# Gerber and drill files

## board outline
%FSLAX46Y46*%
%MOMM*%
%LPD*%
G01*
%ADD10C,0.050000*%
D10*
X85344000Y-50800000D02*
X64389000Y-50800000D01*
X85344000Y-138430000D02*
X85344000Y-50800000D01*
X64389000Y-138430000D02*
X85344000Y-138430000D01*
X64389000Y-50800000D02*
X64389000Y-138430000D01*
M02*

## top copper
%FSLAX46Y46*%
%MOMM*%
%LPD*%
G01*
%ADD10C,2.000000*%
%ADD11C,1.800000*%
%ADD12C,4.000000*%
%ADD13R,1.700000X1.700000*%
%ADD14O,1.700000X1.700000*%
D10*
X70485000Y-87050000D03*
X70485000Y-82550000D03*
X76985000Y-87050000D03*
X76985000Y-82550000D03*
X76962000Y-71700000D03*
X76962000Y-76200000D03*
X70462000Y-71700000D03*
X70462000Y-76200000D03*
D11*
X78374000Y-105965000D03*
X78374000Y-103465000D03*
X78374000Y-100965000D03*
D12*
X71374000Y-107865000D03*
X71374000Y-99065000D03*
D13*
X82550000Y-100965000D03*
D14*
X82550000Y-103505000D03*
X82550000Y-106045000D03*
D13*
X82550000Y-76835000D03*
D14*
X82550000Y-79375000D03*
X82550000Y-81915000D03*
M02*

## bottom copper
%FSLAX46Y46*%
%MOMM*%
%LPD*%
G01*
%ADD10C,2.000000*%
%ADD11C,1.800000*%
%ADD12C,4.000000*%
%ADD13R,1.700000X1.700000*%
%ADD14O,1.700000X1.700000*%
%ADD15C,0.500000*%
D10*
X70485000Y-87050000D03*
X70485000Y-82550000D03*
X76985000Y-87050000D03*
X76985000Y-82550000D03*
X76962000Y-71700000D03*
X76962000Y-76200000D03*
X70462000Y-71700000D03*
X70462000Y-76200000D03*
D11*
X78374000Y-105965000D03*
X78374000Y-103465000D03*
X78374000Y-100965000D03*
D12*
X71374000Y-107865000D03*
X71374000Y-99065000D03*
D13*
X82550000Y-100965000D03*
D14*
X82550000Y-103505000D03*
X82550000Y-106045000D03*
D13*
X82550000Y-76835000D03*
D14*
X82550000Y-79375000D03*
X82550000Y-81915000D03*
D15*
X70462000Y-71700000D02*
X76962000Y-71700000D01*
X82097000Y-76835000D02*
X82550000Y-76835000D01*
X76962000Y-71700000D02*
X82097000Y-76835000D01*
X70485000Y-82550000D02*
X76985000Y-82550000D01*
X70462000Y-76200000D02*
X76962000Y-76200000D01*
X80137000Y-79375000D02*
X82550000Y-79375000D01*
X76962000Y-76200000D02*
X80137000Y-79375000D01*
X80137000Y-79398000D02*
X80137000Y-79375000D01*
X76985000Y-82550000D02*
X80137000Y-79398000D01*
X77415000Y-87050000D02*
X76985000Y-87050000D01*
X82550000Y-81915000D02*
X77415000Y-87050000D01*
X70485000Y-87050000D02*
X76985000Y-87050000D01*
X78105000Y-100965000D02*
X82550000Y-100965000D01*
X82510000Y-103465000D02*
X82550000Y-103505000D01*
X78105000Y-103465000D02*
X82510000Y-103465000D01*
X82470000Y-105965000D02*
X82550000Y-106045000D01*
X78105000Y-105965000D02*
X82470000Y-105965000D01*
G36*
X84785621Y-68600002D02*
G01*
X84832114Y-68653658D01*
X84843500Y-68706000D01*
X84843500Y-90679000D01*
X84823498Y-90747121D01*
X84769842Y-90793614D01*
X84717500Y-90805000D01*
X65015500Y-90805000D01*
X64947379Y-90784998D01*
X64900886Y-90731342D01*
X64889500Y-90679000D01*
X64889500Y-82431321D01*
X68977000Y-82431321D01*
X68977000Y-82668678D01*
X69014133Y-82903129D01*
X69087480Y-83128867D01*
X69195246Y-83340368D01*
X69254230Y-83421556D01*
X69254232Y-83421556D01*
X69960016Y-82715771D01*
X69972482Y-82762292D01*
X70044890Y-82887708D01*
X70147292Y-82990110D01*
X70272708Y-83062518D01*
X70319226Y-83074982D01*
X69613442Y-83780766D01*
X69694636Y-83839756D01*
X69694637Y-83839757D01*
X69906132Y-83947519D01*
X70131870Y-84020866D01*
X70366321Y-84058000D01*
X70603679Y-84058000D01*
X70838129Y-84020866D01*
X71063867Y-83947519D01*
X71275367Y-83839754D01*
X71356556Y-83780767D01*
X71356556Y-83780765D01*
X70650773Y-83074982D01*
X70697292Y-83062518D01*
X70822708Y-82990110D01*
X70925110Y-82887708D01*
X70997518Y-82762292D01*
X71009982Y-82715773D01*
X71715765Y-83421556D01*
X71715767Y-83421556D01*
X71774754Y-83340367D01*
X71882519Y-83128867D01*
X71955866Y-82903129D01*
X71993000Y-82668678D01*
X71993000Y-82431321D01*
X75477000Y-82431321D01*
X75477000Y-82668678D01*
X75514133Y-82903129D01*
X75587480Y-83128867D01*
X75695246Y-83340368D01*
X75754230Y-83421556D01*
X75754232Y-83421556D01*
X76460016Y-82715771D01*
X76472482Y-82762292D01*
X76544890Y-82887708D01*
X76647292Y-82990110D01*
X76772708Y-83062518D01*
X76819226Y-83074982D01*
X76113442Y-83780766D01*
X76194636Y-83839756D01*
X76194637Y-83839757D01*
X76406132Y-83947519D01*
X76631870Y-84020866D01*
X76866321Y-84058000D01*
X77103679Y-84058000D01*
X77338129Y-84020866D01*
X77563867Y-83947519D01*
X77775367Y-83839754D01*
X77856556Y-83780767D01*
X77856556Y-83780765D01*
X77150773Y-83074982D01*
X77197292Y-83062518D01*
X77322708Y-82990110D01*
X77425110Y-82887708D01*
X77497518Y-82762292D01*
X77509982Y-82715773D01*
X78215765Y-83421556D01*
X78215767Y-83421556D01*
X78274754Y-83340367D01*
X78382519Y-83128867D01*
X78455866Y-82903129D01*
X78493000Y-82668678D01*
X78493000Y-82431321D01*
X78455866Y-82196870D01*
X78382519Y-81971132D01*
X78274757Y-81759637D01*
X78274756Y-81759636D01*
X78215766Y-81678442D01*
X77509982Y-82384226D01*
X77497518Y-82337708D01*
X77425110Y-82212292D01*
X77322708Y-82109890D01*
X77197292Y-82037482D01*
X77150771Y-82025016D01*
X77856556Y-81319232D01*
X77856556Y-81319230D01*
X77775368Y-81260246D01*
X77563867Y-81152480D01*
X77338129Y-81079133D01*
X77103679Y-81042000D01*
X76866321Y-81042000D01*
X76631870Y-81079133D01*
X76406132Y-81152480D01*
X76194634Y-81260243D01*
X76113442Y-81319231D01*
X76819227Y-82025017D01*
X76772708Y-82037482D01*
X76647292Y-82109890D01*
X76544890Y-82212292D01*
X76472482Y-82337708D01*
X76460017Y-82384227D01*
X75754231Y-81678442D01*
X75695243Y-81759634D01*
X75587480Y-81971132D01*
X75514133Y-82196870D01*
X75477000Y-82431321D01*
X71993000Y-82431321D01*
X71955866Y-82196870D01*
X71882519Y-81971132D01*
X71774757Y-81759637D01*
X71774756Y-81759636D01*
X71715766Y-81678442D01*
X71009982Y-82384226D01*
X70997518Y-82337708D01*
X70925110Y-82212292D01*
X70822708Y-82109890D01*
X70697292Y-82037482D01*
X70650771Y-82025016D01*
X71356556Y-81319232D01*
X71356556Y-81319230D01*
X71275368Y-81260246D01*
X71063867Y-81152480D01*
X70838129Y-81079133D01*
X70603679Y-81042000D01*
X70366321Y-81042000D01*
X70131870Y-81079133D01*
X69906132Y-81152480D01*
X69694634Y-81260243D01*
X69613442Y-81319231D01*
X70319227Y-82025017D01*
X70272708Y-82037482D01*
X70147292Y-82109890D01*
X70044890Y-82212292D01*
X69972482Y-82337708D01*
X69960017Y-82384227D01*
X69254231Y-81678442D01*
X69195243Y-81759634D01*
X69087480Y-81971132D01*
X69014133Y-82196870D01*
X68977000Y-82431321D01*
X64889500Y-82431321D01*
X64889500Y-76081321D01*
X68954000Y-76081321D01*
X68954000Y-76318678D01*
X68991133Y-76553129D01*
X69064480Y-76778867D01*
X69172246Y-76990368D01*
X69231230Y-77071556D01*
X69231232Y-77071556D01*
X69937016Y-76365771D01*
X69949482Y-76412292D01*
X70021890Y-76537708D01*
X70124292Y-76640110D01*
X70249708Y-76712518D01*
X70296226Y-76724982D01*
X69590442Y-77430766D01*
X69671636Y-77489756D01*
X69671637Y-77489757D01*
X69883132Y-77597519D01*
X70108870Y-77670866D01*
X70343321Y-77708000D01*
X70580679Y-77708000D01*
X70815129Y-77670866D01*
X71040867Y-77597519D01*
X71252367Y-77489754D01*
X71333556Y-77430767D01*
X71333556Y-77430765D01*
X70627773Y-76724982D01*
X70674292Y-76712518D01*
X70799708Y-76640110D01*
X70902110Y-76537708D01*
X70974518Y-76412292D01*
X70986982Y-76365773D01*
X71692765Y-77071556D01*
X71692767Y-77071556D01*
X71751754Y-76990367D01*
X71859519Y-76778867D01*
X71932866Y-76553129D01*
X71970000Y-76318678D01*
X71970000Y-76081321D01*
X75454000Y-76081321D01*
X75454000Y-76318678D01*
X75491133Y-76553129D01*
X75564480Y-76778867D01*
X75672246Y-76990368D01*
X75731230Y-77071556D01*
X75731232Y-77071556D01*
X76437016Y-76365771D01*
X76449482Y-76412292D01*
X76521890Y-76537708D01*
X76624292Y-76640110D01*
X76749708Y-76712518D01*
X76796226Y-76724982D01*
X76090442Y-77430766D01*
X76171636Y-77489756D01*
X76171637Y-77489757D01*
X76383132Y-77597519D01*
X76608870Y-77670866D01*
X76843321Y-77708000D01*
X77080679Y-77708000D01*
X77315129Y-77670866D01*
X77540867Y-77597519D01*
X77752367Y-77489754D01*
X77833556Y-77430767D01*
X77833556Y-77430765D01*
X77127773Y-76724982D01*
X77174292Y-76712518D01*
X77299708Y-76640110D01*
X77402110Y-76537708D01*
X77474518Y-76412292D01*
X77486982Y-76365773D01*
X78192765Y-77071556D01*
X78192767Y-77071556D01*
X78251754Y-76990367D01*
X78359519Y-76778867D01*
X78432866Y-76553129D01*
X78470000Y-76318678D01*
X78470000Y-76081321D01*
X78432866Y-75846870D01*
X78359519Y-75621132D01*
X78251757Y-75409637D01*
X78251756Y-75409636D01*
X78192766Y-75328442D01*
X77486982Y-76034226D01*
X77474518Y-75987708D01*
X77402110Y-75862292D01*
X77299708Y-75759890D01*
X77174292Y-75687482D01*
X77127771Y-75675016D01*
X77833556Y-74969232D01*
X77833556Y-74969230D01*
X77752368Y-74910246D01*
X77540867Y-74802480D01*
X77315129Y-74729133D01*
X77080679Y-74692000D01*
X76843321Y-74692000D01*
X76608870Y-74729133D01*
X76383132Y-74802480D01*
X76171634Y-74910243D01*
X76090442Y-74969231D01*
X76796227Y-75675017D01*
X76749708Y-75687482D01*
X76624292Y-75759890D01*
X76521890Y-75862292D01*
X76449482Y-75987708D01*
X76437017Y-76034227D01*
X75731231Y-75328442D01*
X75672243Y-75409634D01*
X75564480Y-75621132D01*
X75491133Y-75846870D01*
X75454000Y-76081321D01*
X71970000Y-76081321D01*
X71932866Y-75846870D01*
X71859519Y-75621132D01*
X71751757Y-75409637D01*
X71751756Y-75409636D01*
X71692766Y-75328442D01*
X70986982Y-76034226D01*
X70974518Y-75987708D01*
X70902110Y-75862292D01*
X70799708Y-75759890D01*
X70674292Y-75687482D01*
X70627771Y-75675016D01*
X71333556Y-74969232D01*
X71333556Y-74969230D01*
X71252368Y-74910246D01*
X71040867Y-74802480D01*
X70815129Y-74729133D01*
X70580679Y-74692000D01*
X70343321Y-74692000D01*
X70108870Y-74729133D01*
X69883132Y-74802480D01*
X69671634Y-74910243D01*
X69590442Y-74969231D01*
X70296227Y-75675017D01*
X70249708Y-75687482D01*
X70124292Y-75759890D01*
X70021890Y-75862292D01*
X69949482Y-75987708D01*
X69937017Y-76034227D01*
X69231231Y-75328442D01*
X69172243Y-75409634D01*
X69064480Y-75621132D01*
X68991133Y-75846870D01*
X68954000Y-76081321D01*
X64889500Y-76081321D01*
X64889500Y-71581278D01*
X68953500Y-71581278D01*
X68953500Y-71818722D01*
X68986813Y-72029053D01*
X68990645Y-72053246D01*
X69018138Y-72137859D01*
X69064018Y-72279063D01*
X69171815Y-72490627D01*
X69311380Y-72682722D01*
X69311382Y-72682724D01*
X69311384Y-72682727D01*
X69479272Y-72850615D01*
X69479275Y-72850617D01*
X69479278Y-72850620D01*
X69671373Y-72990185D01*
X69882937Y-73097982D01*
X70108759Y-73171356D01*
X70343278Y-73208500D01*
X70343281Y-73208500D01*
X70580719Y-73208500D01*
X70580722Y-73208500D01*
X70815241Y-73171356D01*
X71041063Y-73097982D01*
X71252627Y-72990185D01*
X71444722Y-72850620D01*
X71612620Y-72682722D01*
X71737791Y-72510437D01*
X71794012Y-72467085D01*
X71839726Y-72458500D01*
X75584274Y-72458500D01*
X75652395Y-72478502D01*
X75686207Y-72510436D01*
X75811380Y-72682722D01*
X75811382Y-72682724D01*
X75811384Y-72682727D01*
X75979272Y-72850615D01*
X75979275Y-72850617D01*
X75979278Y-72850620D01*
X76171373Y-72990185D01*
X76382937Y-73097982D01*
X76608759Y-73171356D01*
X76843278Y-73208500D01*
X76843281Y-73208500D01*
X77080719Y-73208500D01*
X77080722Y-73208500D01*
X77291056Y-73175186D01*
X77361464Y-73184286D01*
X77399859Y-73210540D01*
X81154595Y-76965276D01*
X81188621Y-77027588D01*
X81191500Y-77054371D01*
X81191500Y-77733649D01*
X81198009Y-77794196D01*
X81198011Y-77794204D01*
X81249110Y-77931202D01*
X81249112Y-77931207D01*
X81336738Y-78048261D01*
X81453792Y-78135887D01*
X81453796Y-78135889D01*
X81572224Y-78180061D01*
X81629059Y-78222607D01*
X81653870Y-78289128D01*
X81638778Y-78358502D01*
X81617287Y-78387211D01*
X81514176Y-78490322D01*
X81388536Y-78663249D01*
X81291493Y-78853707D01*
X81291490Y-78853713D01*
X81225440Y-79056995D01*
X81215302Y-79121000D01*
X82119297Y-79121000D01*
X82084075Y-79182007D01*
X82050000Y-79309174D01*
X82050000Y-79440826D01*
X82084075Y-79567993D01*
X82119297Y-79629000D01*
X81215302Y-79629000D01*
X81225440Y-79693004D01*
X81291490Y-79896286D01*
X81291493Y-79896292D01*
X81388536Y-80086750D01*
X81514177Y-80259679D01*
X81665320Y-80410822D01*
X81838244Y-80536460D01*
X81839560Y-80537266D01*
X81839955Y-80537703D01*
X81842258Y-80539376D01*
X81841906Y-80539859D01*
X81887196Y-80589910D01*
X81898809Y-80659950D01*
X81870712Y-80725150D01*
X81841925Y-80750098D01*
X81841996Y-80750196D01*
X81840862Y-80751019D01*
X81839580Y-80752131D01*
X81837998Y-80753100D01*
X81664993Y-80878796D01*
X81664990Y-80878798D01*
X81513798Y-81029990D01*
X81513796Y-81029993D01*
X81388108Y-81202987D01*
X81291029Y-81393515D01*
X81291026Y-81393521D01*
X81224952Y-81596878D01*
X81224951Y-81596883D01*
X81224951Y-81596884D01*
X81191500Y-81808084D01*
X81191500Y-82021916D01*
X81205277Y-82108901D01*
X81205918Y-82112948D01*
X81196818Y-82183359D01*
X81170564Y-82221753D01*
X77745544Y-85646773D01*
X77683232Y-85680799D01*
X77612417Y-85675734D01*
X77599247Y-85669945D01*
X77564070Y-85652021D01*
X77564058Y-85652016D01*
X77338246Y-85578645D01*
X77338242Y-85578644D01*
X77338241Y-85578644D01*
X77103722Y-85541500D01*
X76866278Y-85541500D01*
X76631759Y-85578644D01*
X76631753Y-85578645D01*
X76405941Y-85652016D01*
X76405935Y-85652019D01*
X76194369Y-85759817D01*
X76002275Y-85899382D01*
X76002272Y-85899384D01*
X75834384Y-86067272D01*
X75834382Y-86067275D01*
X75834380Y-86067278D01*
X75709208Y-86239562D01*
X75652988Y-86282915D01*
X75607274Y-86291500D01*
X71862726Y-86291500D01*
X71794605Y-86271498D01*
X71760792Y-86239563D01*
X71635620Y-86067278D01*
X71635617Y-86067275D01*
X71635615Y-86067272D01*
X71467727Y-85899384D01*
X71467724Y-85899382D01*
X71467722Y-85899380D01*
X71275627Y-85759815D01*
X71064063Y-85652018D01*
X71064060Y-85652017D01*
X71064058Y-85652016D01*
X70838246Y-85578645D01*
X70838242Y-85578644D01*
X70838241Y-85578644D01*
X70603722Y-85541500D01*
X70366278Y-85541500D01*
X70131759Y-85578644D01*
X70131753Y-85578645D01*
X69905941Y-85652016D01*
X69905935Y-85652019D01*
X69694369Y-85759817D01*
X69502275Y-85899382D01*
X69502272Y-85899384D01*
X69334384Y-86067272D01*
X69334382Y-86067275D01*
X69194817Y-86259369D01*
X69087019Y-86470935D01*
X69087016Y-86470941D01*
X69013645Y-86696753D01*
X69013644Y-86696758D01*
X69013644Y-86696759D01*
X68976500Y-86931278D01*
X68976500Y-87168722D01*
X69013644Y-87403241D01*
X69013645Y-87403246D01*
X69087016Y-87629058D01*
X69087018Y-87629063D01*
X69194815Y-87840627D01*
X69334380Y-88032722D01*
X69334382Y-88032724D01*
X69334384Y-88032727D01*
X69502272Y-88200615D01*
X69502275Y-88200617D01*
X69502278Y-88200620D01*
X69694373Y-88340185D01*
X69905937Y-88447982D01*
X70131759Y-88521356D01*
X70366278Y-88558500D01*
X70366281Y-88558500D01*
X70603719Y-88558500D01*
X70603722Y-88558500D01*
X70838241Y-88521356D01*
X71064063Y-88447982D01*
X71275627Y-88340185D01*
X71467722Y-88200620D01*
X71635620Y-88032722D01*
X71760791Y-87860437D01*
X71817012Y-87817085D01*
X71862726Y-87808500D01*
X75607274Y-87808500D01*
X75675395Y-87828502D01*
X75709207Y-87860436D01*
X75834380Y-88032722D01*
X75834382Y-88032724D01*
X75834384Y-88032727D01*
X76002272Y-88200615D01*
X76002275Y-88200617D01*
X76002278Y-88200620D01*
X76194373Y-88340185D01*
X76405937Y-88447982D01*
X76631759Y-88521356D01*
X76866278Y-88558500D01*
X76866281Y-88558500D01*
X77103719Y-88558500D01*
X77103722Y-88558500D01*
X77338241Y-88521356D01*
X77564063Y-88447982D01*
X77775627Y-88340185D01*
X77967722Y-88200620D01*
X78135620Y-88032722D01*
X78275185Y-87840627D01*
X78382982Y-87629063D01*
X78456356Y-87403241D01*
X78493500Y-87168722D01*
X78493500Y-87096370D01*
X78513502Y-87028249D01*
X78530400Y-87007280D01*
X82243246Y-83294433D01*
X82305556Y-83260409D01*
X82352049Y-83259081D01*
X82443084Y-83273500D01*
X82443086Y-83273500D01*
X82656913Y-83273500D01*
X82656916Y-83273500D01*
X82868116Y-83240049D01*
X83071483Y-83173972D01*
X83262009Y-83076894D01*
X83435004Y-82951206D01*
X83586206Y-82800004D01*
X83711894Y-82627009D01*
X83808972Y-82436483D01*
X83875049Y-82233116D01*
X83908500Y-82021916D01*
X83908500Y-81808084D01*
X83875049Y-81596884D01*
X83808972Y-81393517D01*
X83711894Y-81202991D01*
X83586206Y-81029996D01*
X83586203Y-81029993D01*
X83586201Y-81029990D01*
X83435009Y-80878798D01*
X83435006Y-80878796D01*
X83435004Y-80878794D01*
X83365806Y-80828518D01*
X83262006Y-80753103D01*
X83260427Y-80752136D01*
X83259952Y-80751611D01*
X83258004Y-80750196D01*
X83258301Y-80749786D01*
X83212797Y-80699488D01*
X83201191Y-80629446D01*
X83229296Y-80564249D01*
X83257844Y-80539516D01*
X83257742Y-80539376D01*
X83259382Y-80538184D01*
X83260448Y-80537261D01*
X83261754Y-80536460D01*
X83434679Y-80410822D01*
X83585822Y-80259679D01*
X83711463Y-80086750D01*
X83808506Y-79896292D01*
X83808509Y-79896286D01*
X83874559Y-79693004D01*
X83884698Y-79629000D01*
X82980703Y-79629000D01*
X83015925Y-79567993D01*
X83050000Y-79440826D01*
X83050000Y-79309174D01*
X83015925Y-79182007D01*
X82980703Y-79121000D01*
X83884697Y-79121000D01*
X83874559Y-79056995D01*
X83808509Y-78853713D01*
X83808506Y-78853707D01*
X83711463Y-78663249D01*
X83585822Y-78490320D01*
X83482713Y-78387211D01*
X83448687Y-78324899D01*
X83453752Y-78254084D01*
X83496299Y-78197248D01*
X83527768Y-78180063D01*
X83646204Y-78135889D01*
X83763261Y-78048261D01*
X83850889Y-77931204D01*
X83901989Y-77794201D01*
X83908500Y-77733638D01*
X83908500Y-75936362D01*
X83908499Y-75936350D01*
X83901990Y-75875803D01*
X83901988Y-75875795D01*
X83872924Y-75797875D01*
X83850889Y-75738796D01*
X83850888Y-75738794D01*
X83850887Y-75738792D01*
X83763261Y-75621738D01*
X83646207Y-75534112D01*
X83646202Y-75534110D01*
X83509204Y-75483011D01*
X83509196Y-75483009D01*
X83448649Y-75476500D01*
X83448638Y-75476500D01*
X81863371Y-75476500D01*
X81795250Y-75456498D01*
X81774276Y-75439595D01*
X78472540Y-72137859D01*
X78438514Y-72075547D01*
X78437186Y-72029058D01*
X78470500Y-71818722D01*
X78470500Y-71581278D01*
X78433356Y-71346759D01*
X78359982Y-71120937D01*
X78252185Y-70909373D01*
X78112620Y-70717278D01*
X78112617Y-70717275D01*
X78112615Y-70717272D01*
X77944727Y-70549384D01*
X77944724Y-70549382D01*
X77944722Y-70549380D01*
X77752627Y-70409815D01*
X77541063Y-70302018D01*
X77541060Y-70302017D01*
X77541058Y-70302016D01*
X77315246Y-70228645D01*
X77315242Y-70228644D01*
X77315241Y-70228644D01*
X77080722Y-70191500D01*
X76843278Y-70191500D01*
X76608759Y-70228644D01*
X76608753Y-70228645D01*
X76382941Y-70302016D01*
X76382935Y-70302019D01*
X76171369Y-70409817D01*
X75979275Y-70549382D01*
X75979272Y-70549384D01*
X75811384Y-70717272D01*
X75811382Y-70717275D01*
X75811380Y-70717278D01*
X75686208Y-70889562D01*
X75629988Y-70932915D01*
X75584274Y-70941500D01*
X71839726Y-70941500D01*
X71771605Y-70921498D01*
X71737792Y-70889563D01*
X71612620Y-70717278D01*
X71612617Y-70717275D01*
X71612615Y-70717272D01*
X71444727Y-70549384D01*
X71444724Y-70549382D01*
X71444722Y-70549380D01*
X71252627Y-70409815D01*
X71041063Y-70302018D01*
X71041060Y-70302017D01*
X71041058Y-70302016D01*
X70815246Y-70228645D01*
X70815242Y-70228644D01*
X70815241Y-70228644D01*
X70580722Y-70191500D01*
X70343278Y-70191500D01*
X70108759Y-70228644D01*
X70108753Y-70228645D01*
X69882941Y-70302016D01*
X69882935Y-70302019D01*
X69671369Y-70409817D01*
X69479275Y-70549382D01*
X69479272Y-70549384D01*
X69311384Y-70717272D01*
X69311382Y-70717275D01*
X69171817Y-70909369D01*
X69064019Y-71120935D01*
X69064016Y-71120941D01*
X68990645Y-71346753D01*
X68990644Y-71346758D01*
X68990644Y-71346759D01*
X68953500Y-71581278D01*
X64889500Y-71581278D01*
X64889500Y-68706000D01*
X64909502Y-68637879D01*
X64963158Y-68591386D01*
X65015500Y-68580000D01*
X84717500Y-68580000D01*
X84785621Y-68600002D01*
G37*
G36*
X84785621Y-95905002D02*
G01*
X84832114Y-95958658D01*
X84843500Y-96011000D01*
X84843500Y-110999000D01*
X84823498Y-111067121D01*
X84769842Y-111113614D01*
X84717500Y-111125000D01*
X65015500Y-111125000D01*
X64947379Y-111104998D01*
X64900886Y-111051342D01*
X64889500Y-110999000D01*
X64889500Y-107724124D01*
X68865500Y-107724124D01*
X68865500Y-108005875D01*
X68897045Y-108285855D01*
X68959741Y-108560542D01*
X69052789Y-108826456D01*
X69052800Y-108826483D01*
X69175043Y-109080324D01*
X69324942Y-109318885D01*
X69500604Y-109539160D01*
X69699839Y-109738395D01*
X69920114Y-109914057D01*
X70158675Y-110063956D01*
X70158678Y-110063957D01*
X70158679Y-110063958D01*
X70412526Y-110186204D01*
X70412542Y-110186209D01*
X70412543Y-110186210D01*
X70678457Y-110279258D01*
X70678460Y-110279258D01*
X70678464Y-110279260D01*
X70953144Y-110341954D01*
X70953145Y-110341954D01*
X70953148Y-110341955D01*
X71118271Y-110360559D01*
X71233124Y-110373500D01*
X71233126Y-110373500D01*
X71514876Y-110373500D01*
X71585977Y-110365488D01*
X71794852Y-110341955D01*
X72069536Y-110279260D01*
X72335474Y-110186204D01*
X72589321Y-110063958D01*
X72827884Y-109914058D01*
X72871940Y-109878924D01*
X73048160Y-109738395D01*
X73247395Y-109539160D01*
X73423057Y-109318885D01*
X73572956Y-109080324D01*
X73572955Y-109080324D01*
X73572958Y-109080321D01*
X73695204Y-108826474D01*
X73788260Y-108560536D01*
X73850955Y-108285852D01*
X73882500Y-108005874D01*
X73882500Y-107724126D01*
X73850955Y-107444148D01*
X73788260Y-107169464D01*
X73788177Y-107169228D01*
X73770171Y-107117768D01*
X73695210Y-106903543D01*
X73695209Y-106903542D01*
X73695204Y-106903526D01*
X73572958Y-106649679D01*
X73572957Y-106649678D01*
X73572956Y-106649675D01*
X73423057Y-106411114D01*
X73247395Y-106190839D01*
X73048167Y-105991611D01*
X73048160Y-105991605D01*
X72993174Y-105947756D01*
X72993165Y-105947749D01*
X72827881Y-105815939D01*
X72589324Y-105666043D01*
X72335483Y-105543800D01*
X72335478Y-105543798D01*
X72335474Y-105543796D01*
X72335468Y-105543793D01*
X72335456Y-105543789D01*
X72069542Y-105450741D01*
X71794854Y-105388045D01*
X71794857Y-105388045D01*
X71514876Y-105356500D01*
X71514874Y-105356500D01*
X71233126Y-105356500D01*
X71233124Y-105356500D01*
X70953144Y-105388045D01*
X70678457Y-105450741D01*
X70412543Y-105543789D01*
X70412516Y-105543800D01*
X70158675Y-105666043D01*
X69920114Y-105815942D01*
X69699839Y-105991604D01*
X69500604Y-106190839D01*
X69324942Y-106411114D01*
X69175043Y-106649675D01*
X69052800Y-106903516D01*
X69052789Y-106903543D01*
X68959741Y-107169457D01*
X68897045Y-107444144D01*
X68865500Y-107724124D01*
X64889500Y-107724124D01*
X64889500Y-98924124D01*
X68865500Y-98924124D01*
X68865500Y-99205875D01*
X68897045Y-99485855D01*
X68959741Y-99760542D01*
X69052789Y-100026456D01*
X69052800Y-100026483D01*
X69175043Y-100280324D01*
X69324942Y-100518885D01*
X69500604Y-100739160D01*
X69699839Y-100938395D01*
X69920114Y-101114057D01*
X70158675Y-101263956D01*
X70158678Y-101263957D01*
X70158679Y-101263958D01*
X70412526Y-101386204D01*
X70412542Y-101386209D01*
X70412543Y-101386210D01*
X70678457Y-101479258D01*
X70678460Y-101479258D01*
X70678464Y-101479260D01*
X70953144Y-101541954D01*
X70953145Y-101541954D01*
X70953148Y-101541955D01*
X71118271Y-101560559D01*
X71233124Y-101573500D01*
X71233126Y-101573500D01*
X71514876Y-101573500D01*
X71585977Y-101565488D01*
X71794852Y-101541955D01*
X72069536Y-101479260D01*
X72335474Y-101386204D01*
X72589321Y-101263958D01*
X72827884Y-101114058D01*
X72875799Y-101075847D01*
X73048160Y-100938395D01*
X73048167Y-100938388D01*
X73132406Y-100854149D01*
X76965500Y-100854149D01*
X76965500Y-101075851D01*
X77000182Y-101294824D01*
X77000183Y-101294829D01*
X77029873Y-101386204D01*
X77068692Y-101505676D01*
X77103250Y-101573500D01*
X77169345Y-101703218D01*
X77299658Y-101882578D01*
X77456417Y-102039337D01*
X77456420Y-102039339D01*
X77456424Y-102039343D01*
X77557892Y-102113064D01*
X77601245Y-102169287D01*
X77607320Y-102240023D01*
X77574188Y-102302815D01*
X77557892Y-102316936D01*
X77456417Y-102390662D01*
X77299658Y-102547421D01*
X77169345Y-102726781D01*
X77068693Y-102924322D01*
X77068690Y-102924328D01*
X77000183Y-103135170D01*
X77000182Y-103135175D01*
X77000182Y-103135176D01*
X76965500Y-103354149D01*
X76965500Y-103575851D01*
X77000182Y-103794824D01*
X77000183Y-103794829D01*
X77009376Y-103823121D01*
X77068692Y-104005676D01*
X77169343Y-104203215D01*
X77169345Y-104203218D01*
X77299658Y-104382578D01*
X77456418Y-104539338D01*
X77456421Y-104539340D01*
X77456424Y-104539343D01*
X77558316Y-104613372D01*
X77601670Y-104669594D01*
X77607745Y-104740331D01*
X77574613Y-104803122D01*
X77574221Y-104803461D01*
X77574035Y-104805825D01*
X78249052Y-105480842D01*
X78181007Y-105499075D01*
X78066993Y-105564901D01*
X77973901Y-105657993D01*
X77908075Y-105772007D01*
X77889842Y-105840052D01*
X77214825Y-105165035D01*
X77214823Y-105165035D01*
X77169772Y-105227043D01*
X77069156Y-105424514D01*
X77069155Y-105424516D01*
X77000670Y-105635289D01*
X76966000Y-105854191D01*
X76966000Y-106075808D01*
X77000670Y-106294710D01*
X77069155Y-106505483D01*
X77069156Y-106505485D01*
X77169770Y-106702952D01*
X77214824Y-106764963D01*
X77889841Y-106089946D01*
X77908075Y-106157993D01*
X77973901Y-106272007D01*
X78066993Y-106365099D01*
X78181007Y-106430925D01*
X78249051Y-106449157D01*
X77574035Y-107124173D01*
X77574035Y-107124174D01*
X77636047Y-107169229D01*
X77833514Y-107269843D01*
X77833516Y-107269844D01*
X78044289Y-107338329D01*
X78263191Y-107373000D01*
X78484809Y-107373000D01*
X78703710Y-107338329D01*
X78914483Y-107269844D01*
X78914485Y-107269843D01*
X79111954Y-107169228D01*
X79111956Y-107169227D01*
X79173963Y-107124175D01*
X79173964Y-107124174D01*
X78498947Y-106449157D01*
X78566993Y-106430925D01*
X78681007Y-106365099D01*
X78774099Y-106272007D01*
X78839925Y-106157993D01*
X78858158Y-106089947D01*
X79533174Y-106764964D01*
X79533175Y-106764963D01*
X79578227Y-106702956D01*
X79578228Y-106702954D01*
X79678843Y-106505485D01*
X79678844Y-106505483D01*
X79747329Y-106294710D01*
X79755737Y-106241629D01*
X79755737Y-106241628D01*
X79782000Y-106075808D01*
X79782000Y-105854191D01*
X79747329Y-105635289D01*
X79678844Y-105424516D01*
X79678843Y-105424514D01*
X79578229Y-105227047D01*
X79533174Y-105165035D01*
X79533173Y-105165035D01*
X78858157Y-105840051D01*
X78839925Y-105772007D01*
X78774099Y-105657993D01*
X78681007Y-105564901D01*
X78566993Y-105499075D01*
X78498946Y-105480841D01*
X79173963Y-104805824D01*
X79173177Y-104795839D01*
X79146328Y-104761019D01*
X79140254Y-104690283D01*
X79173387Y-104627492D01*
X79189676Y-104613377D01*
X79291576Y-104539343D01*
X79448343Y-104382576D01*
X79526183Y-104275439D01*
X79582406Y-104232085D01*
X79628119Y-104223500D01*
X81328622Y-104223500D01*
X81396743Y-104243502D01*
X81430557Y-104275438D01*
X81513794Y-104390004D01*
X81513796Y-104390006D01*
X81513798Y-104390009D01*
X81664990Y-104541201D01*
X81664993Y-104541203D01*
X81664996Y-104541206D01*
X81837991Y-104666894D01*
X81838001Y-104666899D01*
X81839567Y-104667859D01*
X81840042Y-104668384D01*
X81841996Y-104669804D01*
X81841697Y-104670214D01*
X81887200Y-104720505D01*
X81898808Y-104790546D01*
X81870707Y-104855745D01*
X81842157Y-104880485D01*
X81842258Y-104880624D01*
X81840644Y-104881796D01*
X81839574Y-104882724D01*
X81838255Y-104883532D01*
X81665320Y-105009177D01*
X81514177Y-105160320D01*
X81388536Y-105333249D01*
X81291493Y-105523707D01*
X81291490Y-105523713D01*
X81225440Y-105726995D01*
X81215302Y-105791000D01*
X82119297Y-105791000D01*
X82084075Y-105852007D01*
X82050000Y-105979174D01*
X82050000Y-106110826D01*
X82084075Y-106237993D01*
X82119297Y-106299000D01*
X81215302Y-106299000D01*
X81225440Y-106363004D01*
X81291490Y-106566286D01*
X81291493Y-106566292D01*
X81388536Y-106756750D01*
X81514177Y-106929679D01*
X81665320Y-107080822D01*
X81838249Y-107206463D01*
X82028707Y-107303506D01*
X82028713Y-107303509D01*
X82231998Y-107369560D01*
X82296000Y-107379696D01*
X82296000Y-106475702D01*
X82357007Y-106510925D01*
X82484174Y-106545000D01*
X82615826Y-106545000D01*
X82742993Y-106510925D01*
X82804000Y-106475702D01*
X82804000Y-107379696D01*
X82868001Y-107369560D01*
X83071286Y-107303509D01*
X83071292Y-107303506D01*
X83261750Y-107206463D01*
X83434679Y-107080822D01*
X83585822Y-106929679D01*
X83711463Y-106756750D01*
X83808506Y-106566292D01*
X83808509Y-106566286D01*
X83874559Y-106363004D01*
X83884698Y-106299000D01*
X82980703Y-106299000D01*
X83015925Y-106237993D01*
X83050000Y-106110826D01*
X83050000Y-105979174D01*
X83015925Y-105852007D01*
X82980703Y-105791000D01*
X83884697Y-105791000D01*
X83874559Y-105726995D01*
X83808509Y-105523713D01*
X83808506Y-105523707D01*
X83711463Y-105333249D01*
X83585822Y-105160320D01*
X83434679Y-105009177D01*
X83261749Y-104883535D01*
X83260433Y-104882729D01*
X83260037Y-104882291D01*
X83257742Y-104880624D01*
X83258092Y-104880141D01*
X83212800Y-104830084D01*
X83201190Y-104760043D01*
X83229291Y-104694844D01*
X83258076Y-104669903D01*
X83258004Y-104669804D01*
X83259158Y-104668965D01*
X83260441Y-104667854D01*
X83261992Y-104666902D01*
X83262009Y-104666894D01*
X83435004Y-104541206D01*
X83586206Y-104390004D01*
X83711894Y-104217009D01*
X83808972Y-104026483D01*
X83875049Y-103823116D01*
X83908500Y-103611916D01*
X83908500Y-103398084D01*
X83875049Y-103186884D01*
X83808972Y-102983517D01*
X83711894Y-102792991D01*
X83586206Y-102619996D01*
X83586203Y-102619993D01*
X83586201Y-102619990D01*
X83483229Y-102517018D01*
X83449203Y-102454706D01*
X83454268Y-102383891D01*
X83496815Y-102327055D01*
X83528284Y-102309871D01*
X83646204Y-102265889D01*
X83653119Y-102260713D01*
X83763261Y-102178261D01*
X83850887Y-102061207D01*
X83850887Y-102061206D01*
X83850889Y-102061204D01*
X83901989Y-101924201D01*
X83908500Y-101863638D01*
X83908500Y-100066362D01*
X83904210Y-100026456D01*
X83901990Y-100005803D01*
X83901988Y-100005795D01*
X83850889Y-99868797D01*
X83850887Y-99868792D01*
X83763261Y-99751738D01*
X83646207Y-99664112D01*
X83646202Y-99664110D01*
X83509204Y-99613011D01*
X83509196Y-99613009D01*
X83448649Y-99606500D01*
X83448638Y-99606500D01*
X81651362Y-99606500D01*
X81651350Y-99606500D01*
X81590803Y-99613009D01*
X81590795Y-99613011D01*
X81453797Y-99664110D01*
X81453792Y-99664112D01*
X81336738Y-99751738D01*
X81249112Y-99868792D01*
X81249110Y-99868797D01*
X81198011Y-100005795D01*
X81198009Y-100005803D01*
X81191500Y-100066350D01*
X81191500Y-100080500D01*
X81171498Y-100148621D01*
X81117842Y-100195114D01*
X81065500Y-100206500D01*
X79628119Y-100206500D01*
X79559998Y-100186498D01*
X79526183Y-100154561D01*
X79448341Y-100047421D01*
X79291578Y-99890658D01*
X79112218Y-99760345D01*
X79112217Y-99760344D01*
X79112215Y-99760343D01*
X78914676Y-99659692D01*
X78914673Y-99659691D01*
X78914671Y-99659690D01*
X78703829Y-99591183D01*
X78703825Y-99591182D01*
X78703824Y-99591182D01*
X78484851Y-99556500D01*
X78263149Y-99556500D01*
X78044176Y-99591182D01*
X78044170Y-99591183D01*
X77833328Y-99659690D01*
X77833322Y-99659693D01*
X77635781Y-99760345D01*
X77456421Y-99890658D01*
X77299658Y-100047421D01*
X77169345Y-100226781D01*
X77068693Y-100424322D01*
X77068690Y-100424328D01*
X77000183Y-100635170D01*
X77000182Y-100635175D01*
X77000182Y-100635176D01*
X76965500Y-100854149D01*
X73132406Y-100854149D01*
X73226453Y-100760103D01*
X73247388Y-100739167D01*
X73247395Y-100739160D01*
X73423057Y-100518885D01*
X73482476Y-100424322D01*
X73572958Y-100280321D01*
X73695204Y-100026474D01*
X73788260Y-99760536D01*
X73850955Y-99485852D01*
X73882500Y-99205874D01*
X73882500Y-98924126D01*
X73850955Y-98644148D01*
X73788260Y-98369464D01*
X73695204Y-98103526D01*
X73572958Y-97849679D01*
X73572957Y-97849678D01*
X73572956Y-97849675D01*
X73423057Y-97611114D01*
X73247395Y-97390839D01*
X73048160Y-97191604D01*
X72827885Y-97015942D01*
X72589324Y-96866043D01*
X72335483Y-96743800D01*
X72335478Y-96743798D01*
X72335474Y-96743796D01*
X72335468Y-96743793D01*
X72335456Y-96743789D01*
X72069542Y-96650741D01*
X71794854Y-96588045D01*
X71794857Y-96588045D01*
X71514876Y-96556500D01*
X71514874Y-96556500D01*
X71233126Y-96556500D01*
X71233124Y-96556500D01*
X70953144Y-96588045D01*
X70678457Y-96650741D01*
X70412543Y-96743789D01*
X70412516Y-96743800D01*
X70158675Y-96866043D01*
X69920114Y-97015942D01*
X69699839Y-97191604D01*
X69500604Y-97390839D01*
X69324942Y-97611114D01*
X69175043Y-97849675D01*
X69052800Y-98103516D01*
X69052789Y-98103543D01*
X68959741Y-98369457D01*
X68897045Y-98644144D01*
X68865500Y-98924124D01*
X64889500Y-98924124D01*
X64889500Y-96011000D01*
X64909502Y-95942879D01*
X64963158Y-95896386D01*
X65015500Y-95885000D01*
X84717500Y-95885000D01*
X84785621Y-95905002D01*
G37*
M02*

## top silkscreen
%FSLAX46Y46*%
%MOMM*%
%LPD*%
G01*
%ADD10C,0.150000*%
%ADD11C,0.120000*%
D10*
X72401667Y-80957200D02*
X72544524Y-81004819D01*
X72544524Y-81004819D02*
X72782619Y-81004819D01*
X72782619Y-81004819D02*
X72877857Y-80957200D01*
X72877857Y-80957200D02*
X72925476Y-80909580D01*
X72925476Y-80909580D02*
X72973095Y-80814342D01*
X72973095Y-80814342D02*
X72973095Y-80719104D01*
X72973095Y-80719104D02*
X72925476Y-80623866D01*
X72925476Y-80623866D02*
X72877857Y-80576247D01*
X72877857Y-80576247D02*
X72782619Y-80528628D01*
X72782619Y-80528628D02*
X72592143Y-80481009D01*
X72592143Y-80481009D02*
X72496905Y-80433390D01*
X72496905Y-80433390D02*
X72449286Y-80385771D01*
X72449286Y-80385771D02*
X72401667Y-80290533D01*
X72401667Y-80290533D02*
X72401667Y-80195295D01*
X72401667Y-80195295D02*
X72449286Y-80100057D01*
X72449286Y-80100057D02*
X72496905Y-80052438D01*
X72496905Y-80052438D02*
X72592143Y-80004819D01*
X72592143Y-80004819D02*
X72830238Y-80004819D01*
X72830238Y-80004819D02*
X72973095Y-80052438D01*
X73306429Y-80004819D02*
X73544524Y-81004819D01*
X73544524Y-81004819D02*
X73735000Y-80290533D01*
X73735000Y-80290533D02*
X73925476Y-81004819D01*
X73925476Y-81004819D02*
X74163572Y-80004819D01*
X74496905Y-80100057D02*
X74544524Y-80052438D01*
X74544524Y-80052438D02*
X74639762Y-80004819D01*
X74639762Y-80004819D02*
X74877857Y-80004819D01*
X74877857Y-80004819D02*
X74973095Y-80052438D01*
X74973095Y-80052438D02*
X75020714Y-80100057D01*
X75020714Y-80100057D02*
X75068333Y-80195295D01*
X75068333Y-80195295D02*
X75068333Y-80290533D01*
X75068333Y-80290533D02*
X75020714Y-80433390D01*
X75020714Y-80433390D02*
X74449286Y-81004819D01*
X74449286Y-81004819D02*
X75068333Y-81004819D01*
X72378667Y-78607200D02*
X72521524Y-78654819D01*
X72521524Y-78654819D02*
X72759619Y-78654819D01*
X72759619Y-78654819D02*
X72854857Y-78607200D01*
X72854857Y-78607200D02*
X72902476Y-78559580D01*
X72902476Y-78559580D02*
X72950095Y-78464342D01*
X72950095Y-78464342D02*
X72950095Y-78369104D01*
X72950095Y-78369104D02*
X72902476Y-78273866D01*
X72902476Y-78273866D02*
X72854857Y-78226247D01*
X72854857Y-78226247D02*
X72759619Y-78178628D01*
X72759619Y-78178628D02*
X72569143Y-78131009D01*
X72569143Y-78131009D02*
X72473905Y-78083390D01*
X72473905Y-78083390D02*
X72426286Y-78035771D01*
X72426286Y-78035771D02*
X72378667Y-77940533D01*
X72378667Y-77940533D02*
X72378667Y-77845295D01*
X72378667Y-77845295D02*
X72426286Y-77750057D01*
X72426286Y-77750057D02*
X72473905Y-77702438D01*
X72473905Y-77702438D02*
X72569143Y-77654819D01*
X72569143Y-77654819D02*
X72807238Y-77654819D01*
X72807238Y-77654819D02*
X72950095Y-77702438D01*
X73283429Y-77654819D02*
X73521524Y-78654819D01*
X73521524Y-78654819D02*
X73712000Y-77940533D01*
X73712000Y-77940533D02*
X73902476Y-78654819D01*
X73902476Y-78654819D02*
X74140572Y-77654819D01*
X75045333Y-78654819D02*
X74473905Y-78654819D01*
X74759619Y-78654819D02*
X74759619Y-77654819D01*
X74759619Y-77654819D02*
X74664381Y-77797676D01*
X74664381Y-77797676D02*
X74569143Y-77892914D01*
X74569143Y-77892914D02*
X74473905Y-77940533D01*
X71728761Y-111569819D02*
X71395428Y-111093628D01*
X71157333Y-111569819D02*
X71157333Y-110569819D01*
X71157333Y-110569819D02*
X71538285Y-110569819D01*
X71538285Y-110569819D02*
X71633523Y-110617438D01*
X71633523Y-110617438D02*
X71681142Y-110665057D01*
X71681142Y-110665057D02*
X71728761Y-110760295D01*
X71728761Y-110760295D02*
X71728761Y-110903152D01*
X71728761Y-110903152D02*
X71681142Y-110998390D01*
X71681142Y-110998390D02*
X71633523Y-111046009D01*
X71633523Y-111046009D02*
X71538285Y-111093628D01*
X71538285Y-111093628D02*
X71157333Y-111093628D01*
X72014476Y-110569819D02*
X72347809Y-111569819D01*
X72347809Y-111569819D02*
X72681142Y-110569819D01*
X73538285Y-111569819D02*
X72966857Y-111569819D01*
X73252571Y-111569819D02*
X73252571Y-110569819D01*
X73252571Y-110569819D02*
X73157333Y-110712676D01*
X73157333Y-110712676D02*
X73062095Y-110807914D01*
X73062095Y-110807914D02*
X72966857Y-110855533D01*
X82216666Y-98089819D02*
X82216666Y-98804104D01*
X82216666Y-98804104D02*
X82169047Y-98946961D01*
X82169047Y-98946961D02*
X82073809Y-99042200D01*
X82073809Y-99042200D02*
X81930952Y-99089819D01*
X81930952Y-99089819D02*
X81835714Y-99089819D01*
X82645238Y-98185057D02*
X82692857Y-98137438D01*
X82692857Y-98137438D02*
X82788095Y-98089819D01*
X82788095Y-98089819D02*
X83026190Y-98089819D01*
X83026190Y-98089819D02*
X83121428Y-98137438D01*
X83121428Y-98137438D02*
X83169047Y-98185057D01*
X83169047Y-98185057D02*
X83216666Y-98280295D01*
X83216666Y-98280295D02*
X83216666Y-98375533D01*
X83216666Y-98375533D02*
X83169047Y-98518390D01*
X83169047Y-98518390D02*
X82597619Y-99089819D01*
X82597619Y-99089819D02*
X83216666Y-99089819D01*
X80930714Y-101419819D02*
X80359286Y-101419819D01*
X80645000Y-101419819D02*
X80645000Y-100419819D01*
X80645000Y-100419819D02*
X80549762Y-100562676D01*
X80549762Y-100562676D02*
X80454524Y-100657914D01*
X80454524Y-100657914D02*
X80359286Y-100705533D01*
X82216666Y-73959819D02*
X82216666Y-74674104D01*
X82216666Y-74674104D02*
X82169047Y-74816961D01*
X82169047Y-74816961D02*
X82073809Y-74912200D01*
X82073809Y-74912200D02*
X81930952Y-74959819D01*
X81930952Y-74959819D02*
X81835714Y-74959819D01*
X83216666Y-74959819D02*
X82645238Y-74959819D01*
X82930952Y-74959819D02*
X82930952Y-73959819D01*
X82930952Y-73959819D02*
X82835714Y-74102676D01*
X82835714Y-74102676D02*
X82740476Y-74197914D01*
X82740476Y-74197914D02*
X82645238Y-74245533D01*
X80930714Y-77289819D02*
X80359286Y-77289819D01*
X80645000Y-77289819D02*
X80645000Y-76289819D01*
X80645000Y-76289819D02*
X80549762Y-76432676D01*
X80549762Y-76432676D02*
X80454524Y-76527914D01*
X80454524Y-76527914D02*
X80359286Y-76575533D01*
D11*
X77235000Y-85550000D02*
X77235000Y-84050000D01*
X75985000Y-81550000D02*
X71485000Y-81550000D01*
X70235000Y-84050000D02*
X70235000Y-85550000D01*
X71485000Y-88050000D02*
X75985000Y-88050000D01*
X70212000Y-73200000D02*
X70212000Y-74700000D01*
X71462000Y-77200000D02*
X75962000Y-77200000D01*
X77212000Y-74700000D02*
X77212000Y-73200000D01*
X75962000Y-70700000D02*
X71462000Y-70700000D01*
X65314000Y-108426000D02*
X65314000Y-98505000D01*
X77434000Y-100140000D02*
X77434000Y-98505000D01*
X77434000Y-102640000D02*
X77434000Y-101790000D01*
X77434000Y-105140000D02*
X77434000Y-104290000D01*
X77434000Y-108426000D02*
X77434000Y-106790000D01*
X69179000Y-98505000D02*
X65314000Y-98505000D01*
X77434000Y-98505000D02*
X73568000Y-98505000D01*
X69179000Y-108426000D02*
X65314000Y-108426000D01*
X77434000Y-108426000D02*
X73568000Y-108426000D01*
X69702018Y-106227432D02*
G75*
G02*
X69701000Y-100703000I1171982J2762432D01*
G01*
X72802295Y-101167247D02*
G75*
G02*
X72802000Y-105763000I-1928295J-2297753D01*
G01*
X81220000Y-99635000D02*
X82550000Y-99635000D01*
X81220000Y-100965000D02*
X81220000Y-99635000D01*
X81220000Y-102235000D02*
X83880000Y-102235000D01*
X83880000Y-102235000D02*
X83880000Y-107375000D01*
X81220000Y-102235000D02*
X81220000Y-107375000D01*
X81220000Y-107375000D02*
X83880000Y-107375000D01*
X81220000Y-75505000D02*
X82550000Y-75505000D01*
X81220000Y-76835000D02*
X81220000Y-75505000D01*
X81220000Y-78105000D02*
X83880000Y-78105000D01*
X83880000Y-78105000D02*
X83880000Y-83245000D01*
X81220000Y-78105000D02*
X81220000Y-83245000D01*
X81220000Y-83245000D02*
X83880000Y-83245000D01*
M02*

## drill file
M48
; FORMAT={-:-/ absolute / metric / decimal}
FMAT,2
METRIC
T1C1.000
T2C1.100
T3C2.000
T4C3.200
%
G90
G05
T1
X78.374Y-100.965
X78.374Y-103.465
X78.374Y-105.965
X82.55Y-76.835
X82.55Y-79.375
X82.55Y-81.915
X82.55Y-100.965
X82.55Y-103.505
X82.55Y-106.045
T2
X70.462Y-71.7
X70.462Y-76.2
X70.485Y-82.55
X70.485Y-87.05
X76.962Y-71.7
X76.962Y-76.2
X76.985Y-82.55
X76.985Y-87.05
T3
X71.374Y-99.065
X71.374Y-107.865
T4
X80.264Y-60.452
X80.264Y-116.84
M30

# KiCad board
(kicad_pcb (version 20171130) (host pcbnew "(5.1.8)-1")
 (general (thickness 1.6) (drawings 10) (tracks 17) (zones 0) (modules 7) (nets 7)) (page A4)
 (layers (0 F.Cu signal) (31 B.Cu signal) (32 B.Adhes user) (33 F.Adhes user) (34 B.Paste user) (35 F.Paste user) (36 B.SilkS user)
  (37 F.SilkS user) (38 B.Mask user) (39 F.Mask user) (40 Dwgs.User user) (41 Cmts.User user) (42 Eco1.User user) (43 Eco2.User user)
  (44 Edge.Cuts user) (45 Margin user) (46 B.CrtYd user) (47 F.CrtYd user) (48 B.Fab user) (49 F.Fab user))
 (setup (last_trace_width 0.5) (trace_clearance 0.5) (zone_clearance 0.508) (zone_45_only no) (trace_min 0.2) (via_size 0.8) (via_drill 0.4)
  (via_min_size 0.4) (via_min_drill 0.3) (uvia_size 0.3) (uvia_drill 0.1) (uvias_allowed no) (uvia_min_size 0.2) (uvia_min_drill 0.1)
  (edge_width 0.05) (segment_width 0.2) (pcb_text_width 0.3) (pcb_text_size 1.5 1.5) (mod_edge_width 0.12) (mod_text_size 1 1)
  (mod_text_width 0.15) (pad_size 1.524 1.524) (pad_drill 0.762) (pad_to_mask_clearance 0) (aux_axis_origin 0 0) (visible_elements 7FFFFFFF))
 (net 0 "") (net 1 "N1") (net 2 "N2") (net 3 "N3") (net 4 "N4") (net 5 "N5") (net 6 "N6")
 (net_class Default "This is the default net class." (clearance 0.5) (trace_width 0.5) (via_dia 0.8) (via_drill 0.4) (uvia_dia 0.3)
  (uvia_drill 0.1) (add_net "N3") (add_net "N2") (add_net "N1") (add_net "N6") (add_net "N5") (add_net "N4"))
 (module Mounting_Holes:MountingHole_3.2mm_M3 (layer F.Cu) (at 80.264 116.84)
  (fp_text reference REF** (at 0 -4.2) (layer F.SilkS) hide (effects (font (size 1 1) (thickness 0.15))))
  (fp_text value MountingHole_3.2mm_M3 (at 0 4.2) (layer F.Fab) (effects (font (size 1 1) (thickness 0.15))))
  (pad 1 np_thru_hole circle (at 0 0) (size 3.2 3.2) (drill 3.2) (layers *.Cu *.Mask)))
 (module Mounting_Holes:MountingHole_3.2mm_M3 (layer F.Cu) (at 80.264 60.452)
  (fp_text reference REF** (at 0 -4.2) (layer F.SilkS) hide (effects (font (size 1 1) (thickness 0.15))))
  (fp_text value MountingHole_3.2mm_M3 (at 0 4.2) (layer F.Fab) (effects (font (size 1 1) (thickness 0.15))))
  (pad 1 np_thru_hole circle (at 0 0) (size 3.2 3.2) (drill 3.2) (layers *.Cu *.Mask)))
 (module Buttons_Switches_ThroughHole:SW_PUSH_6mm (layer F.Cu) (at 70.485 82.55)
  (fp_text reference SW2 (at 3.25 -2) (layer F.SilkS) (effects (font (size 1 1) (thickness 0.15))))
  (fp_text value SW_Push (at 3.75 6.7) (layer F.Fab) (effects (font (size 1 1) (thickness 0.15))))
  (fp_line (start 6.75 3) (end 6.75 1.5) (layer F.SilkS) (width 0.12))
  (fp_line (start 5.5 -1) (end 1 -1) (layer F.SilkS) (width 0.12))
  (fp_line (start -0.25 1.5) (end -0.25 3) (layer F.SilkS) (width 0.12))
  (fp_line (start 1 5.5) (end 5.5 5.5) (layer F.SilkS) (width 0.12))
  (pad 2 thru_hole circle (at 0 4.5 90) (size 2 2) (drill 1.1) (layers *.Cu *.Mask) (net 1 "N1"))
  (pad 1 thru_hole circle (at 0 0 90) (size 2 2) (drill 1.1) (layers *.Cu *.Mask) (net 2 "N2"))
  (pad 2 thru_hole circle (at 6.5 4.5 90) (size 2 2) (drill 1.1) (layers *.Cu *.Mask) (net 1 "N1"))
  (pad 1 thru_hole circle (at 6.5 0 90) (size 2 2) (drill 1.1) (layers *.Cu *.Mask) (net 2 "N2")))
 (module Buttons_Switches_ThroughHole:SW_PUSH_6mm (layer F.Cu) (at 76.962 76.2 180)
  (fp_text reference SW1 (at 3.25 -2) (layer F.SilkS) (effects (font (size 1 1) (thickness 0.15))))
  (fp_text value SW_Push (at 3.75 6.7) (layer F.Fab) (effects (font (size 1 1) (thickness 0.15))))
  (fp_line (start 6.75 3) (end 6.75 1.5) (layer F.SilkS) (width 0.12))
  (fp_line (start 5.5 -1) (end 1 -1) (layer F.SilkS) (width 0.12))
  (fp_line (start -0.25 1.5) (end -0.25 3) (layer F.SilkS) (width 0.12))
  (fp_line (start 1 5.5) (end 5.5 5.5) (layer F.SilkS) (width 0.12))
  (pad 2 thru_hole circle (at 0 4.5 270) (size 2 2) (drill 1.1) (layers *.Cu *.Mask) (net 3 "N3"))
  (pad 1 thru_hole circle (at 0 0 270) (size 2 2) (drill 1.1) (layers *.Cu *.Mask) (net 2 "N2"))
  (pad 2 thru_hole circle (at 6.5 4.5 270) (size 2 2) (drill 1.1) (layers *.Cu *.Mask) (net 3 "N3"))
  (pad 1 thru_hole circle (at 6.5 0 270) (size 2 2) (drill 1.1) (layers *.Cu *.Mask) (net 2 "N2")))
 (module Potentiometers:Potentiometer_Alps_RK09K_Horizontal (layer F.Cu) (at 78.374 100.965 180)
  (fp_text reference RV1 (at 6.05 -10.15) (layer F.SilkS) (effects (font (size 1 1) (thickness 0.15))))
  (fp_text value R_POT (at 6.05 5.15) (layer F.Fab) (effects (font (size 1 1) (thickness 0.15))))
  (fp_line (start 13.06 -7.461) (end 13.06 2.46) (layer F.SilkS) (width 0.12))
  (fp_line (start 0.94 0.825) (end 0.94 2.46) (layer F.SilkS) (width 0.12))
  (fp_line (start 0.94 -1.675) (end 0.94 -0.825) (layer F.SilkS) (width 0.12))
  (fp_line (start 0.94 -4.175) (end 0.94 -3.325) (layer F.SilkS) (width 0.12))
  (fp_line (start 0.94 -7.461) (end 0.94 -5.825) (layer F.SilkS) (width 0.12))
  (fp_line (start 9.195 2.46) (end 13.06 2.46) (layer F.SilkS) (width 0.12))
  (fp_line (start 0.94 2.46) (end 4.806 2.46) (layer F.SilkS) (width 0.12))
  (fp_line (start 9.195 -7.461) (end 13.06 -7.461) (layer F.SilkS) (width 0.12))
  (fp_line (start 0.94 -7.461) (end 4.806 -7.461) (layer F.SilkS) (width 0.12))
  (fp_arc (start 7.5 -2.5) (end 8.673 0.262) (angle -134) (layer F.SilkS) (width 0.12))
  (fp_arc (start 7.5 -2.5) (end 5.572 -4.798) (angle -100) (layer F.SilkS) (width 0.12))
  (pad 3 thru_hole circle (at 0 -5 180) (size 1.8 1.8) (drill 1) (layers *.Cu *.Mask) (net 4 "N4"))
  (pad 2 thru_hole circle (at 0 -2.5 180) (size 1.8 1.8) (drill 1) (layers *.Cu *.Mask) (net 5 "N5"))
  (pad 1 thru_hole circle (at 0 0 180) (size 1.8 1.8) (drill 1) (layers *.Cu *.Mask) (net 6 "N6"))
  (pad 0 np_thru_hole circle (at 7 -6.9 180) (size 4 4) (drill 2) (layers *.Cu *.Mask))
  (pad 0 np_thru_hole circle (at 7 1.9 180) (size 4 4) (drill 2) (layers *.Cu *.Mask)))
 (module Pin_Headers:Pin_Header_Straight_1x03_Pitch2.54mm (layer F.Cu) (at 82.55 100.965)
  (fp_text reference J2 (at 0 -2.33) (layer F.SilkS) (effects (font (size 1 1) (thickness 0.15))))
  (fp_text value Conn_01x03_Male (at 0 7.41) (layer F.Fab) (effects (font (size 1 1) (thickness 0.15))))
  (fp_line (start -1.33 -1.33) (end 0 -1.33) (layer F.SilkS) (width 0.12))
  (fp_line (start -1.33 0) (end -1.33 -1.33) (layer F.SilkS) (width 0.12))
  (fp_line (start -1.33 1.27) (end 1.33 1.27) (layer F.SilkS) (width 0.12))
  (fp_line (start 1.33 1.27) (end 1.33 6.41) (layer F.SilkS) (width 0.12))
  (fp_line (start -1.33 1.27) (end -1.33 6.41) (layer F.SilkS) (width 0.12))
  (fp_line (start -1.33 6.41) (end 1.33 6.41) (layer F.SilkS) (width 0.12))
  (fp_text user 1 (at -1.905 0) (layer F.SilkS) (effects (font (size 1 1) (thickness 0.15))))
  (pad 1 thru_hole rect (at 0 0) (size 1.7 1.7) (drill 1) (layers *.Cu *.Mask) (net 6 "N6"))
  (pad 2 thru_hole oval (at 0 2.54) (size 1.7 1.7) (drill 1) (layers *.Cu *.Mask) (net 5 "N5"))
  (pad 3 thru_hole oval (at 0 5.08) (size 1.7 1.7) (drill 1) (layers *.Cu *.Mask) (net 4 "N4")))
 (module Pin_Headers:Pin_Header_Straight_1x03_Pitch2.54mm (layer F.Cu) (at 82.55 76.835)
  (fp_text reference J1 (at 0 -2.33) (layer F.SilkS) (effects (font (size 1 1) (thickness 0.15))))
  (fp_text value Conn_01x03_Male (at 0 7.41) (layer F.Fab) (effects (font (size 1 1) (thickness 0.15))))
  (fp_line (start -1.33 -1.33) (end 0 -1.33) (layer F.SilkS) (width 0.12))
  (fp_line (start -1.33 0) (end -1.33 -1.33) (layer F.SilkS) (width 0.12))
  (fp_line (start -1.33 1.27) (end 1.33 1.27) (layer F.SilkS) (width 0.12))
  (fp_line (start 1.33 1.27) (end 1.33 6.41) (layer F.SilkS) (width 0.12))
  (fp_line (start -1.33 1.27) (end -1.33 6.41) (layer F.SilkS) (width 0.12))
  (fp_line (start -1.33 6.41) (end 1.33 6.41) (layer F.SilkS) (width 0.12))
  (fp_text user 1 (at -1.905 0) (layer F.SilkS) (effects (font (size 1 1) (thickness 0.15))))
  (pad 1 thru_hole rect (at 0 0) (size 1.7 1.7) (drill 1) (layers *.Cu *.Mask) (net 3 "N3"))
  (pad 2 thru_hole oval (at 0 2.54) (size 1.7 1.7) (drill 1) (layers *.Cu *.Mask) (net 2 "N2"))
  (pad 3 thru_hole oval (at 0 5.08) (size 1.7 1.7) (drill 1) (layers *.Cu *.Mask) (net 1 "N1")))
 (gr_line (start 85.344 50.8) (end 64.389 50.8) (layer Edge.Cuts) (width 0.05))
 (gr_line (start 85.344 138.43) (end 85.344 50.8) (layer Edge.Cuts) (width 0.05))
 (gr_line (start 64.389 138.43) (end 85.344 138.43) (layer Edge.Cuts) (width 0.05))
 (gr_line (start 64.389 50.8) (end 64.389 138.43) (layer Edge.Cuts) (width 0.05))
 (segment (start 70.462 71.7) (end 76.962 71.7) (width 0.5) (layer B.Cu) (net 3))
 (segment (start 82.097 76.835) (end 82.55 76.835) (width 0.5) (layer B.Cu) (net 3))
 (segment (start 76.962 71.7) (end 82.097 76.835) (width 0.5) (layer B.Cu) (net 3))
 (segment (start 70.485 82.55) (end 76.985 82.55) (width 0.5) (layer B.Cu) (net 2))
 (segment (start 70.462 76.2) (end 76.962 76.2) (width 0.5) (layer B.Cu) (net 2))
 (segment (start 80.137 79.375) (end 82.55 79.375) (width 0.5) (layer B.Cu) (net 2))
 (segment (start 76.962 76.2) (end 80.137 79.375) (width 0.5) (layer B.Cu) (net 2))
 (segment (start 80.137 79.398) (end 80.137 79.375) (width 0.5) (layer B.Cu) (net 2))
 (segment (start 76.985 82.55) (end 80.137 79.398) (width 0.5) (layer B.Cu) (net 2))
 (segment (start 77.415 87.05) (end 76.985 87.05) (width 0.5) (layer B.Cu) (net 1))
 (segment (start 82.55 81.915) (end 77.415 87.05) (width 0.5) (layer B.Cu) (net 1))
 (segment (start 70.485 87.05) (end 76.985 87.05) (width 0.5) (layer B.Cu) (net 1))
 (segment (start 78.105 100.965) (end 82.55 100.965) (width 0.5) (layer B.Cu) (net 6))
 (segment (start 82.51 103.465) (end 82.55 103.505) (width 0.5) (layer B.Cu) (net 5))
 (segment (start 78.105 103.465) (end 82.51 103.465) (width 0.5) (layer B.Cu) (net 5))
 (segment (start 82.47 105.965) (end 82.55 106.045) (width 0.5) (layer B.Cu) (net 4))
 (segment (start 78.105 105.965) (end 82.47 105.965) (width 0.5) (layer B.Cu) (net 4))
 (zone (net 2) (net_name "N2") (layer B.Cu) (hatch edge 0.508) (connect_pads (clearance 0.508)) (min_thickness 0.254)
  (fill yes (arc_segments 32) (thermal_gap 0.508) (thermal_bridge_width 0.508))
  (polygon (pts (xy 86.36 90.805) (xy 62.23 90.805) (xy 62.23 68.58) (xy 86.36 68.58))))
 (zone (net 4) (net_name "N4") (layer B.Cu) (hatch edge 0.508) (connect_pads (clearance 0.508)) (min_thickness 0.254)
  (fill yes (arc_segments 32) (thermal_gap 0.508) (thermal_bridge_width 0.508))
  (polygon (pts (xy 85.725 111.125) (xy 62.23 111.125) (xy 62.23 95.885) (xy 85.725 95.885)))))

